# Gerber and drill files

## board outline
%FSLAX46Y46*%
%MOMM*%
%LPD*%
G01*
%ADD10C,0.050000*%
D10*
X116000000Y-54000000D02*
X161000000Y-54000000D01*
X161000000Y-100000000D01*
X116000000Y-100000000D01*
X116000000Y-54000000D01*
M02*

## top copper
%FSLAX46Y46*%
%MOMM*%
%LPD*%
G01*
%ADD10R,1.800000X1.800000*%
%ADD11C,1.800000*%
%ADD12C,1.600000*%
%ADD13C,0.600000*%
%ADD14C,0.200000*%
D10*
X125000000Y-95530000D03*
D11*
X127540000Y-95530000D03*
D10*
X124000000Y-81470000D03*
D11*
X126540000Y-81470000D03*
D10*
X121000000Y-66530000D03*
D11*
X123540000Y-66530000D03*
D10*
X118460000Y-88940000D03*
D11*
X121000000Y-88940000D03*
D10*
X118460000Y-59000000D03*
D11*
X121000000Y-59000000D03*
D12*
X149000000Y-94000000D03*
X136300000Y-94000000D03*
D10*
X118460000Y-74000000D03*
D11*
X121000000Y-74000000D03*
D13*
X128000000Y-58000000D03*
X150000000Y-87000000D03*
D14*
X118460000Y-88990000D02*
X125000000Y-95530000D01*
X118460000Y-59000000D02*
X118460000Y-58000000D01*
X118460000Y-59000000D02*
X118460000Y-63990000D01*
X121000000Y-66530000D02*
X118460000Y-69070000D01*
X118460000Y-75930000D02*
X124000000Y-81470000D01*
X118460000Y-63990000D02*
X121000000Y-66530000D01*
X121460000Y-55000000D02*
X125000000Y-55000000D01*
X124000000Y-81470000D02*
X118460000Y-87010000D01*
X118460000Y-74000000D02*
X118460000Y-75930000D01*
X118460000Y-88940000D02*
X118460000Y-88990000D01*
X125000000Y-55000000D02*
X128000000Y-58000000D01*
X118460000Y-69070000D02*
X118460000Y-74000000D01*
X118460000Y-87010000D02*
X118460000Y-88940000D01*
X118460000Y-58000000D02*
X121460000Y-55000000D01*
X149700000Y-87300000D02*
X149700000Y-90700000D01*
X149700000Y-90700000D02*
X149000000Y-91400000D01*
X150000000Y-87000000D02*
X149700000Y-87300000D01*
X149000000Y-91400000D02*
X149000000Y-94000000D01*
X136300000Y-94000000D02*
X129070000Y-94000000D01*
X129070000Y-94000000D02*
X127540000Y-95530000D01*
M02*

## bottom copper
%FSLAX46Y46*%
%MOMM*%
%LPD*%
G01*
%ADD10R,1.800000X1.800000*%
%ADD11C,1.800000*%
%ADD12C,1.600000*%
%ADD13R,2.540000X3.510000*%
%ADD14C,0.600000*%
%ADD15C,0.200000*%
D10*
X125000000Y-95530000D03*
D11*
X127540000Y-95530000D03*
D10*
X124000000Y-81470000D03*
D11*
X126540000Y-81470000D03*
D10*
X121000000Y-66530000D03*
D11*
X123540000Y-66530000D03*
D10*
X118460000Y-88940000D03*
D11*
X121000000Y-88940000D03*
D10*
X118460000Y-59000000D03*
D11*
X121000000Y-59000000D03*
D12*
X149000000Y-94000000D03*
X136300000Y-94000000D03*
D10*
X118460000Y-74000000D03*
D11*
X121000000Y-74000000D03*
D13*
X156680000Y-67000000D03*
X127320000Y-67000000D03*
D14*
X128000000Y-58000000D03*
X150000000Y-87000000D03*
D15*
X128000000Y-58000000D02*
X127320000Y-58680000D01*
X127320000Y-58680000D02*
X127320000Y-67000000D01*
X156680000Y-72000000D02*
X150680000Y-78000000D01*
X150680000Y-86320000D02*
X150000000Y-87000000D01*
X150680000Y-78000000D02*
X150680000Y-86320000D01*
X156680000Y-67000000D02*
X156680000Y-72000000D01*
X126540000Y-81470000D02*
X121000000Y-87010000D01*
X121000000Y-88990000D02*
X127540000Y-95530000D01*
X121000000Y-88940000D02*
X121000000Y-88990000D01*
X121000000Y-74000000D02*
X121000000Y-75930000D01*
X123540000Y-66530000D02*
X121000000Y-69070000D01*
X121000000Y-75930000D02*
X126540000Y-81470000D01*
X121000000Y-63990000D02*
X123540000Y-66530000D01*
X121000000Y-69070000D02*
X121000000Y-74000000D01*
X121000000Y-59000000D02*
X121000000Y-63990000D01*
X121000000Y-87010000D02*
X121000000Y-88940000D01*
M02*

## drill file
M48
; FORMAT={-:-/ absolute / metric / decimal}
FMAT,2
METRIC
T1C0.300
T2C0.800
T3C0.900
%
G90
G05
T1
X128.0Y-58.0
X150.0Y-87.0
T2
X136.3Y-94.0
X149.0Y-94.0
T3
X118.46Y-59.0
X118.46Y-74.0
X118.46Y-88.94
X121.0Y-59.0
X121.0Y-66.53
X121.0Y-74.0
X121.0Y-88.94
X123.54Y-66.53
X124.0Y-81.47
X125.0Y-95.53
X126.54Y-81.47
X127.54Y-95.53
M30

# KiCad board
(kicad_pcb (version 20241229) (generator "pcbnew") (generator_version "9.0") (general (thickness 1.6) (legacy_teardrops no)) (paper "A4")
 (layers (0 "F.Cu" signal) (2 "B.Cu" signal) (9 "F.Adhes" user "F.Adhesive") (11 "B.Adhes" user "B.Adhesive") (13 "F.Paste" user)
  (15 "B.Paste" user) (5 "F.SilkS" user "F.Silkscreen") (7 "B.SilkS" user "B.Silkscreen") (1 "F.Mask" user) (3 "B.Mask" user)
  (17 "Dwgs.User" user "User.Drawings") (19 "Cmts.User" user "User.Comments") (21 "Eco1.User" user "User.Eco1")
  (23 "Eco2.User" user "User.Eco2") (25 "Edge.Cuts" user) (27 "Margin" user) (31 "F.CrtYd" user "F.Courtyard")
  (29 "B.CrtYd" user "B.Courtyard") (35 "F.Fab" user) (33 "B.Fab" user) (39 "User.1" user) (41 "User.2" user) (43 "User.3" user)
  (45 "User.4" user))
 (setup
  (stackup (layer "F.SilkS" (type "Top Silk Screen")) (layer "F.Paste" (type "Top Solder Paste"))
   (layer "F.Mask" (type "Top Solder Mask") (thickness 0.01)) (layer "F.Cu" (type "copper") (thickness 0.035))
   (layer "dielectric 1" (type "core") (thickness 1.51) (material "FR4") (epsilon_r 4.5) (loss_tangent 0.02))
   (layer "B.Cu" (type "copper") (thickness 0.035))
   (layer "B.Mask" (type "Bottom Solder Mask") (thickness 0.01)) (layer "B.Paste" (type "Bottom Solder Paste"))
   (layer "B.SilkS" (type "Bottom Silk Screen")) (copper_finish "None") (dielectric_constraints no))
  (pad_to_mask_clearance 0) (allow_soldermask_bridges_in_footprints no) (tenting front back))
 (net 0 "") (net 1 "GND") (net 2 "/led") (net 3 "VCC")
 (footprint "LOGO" (layer "F.Cu") (at 142 67)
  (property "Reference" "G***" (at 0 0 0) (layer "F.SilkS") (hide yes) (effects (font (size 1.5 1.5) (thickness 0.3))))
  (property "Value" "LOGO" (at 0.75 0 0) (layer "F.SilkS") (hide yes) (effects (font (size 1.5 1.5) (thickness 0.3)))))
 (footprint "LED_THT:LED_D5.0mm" (layer "F.Cu") (at 125 95.53)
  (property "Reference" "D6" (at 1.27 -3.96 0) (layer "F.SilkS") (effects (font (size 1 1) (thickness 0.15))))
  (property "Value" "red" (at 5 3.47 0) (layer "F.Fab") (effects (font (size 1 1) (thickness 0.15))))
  (pad "1" thru_hole rect (at 0 0) (size 1.8 1.8) (drill 0.9) (layers "*.Cu" "*.Mask") (remove_unused_layers no) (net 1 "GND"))
  (pad "2" thru_hole circle (at 2.54 0) (size 1.8 1.8) (drill 0.9) (layers "*.Cu" "*.Mask") (remove_unused_layers no) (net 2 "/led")))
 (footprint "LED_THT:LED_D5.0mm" (layer "F.Cu") (at 124 81.47)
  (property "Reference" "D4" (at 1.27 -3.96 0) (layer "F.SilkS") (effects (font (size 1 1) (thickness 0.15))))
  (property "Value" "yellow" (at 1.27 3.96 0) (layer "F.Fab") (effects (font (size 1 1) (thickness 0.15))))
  (pad "1" thru_hole rect (at 0 0) (size 1.8 1.8) (drill 0.9) (layers "*.Cu" "*.Mask") (remove_unused_layers no) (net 1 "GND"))
  (pad "2" thru_hole circle (at 2.54 0) (size 1.8 1.8) (drill 0.9) (layers "*.Cu" "*.Mask") (remove_unused_layers no) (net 2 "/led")))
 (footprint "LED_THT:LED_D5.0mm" (layer "F.Cu") (at 121 66.53)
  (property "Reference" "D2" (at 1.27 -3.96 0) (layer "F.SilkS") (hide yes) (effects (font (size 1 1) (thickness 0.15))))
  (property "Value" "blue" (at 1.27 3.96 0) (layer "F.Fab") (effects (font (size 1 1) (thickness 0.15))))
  (pad "1" thru_hole rect (at 0 0) (size 1.8 1.8) (drill 0.9) (layers "*.Cu" "*.Mask") (remove_unused_layers no) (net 1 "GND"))
  (pad "2" thru_hole circle (at 2.54 0) (size 1.8 1.8) (drill 0.9) (layers "*.Cu" "*.Mask") (remove_unused_layers no) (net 2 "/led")))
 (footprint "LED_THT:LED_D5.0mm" (layer "F.Cu") (at 118.46 88.94)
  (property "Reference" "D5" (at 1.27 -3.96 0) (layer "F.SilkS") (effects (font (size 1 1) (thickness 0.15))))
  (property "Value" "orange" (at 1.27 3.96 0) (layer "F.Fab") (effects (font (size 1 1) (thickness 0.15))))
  (pad "1" thru_hole rect (at 0 0) (size 1.8 1.8) (drill 0.9) (layers "*.Cu" "*.Mask") (remove_unused_layers no) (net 1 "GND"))
  (pad "2" thru_hole circle (at 2.54 0) (size 1.8 1.8) (drill 0.9) (layers "*.Cu" "*.Mask") (remove_unused_layers no) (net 2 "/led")))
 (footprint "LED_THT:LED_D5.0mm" (layer "F.Cu") (at 118.46 59)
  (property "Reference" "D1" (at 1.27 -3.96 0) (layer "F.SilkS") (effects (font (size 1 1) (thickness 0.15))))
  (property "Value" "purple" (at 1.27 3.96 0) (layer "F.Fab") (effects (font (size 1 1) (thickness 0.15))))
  (pad "1" thru_hole rect (at 0 0) (size 1.8 1.8) (drill 0.9) (layers "*.Cu" "*.Mask") (remove_unused_layers no) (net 1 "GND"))
  (pad "2" thru_hole circle (at 2.54 0) (size 1.8 1.8) (drill 0.9) (layers "*.Cu" "*.Mask") (remove_unused_layers no) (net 2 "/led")))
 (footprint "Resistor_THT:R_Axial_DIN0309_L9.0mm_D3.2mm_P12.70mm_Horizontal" (layer "F.Cu") (at 149 94 180)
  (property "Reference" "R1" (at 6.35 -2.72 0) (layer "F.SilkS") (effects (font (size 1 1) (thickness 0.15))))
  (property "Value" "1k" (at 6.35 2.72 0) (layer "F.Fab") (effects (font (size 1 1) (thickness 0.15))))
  (pad "1" thru_hole circle (at 0 0 180) (size 1.6 1.6) (drill 0.8) (layers "*.Cu" "*.Mask") (remove_unused_layers no) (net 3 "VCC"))
  (pad "2" thru_hole circle (at 12.7 0 180) (size 1.6 1.6) (drill 0.8) (layers "*.Cu" "*.Mask") (remove_unused_layers no) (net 2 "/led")))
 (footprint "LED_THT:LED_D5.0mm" (layer "F.Cu") (at 118.46 74)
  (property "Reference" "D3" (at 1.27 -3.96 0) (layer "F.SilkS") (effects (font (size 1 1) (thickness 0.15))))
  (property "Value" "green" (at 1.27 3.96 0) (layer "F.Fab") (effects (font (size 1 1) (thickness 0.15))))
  (pad "1" thru_hole rect (at 0 0) (size 1.8 1.8) (drill 0.9) (layers "*.Cu" "*.Mask") (remove_unused_layers no) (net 1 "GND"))
  (pad "2" thru_hole circle (at 2.54 0) (size 1.8 1.8) (drill 0.9) (layers "*.Cu" "*.Mask") (remove_unused_layers no) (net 2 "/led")))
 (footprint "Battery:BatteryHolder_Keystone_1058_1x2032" (layer "B.Cu") (at 142 67 180)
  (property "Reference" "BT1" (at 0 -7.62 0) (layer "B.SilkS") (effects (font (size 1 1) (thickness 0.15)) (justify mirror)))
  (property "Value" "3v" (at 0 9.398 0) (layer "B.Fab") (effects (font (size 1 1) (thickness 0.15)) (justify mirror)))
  (pad "1" smd rect (at -14.68 0 180) (size 2.54 3.51) (layers "B.Cu" "B.Mask" "B.Paste") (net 3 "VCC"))
  (pad "2" smd rect (at 14.68 0 180) (size 2.54 3.51) (layers "B.Cu" "B.Mask" "B.Paste") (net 1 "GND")))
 (gr_rect (start 116 54) (end 161 100) (stroke (width 0.05) (type default)) (fill no) (layer "Edge.Cuts"))
 (segment (start 118.46 88.99) (end 125 95.53) (width 0.2) (layer "F.Cu") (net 1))
 (segment (start 118.46 59) (end 118.46 58) (width 0.2) (layer "F.Cu") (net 1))
 (segment (start 118.46 59) (end 118.46 63.99) (width 0.2) (layer "F.Cu") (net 1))
 (segment (start 121 66.53) (end 118.46 69.07) (width 0.2) (layer "F.Cu") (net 1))
 (segment (start 118.46 75.93) (end 124 81.47) (width 0.2) (layer "F.Cu") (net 1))
 (segment (start 118.46 63.99) (end 121 66.53) (width 0.2) (layer "F.Cu") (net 1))
 (segment (start 121.46 55) (end 125 55) (width 0.2) (layer "F.Cu") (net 1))
 (segment (start 124 81.47) (end 118.46 87.01) (width 0.2) (layer "F.Cu") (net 1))
 (segment (start 118.46 74) (end 118.46 75.93) (width 0.2) (layer "F.Cu") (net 1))
 (segment (start 118.46 88.94) (end 118.46 88.99) (width 0.2) (layer "F.Cu") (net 1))
 (segment (start 125 55) (end 128 58) (width 0.2) (layer "F.Cu") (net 1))
 (segment (start 118.46 69.07) (end 118.46 74) (width 0.2) (layer "F.Cu") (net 1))
 (segment (start 118.46 87.01) (end 118.46 88.94) (width 0.2) (layer "F.Cu") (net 1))
 (segment (start 118.46 58) (end 121.46 55) (width 0.2) (layer "F.Cu") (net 1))
 (via (at 128 58) (size 0.6) (drill 0.3) (layers "F.Cu" "B.Cu") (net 1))
 (segment (start 128 58) (end 127.32 58.68) (width 0.2) (layer "B.Cu") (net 1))
 (segment (start 127.32 58.68) (end 127.32 67) (width 0.2) (layer "B.Cu") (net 1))
 (segment (start 149.7 87.3) (end 149.7 90.7) (width 0.2) (layer "F.Cu") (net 3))
 (segment (start 149.7 90.7) (end 149 91.4) (width 0.2) (layer "F.Cu") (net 3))
 (segment (start 150 87) (end 149.7 87.3) (width 0.2) (layer "F.Cu") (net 3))
 (segment (start 149 91.4) (end 149 94) (width 0.2) (layer "F.Cu") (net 3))
 (via (at 150 87) (size 0.6) (drill 0.3) (layers "F.Cu" "B.Cu") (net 3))
 (segment (start 156.68 72) (end 150.68 78) (width 0.2) (layer "B.Cu") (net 3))
 (segment (start 150.68 86.32) (end 150 87) (width 0.2) (layer "B.Cu") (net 3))
 (segment (start 150.68 78) (end 150.68 86.32) (width 0.2) (layer "B.Cu") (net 3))
 (segment (start 156.68 67) (end 156.68 72) (width 0.2) (layer "B.Cu") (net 3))
 (segment (start 136.3 94) (end 129.07 94) (width 0.2) (layer "F.Cu") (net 2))
 (segment (start 129.07 94) (end 127.54 95.53) (width 0.2) (layer "F.Cu") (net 2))
 (segment (start 126.54 81.47) (end 121 87.01) (width 0.2) (layer "B.Cu") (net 2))
 (segment (start 121 88.99) (end 127.54 95.53) (width 0.2) (layer "B.Cu") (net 2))
 (segment (start 121 88.94) (end 121 88.99) (width 0.2) (layer "B.Cu") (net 2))
 (segment (start 121 74) (end 121 75.93) (width 0.2) (layer "B.Cu") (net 2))
 (segment (start 123.54 66.53) (end 121 69.07) (width 0.2) (layer "B.Cu") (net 2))
 (segment (start 121 75.93) (end 126.54 81.47) (width 0.2) (layer "B.Cu") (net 2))
 (segment (start 121 63.99) (end 123.54 66.53) (width 0.2) (layer "B.Cu") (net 2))
 (segment (start 121 69.07) (end 121 74) (width 0.2) (layer "B.Cu") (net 2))
 (segment (start 121 59) (end 121 63.99) (width 0.2) (layer "B.Cu") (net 2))
 (segment (start 121 87.01) (end 121 88.94) (width 0.2) (layer "B.Cu") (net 2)))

